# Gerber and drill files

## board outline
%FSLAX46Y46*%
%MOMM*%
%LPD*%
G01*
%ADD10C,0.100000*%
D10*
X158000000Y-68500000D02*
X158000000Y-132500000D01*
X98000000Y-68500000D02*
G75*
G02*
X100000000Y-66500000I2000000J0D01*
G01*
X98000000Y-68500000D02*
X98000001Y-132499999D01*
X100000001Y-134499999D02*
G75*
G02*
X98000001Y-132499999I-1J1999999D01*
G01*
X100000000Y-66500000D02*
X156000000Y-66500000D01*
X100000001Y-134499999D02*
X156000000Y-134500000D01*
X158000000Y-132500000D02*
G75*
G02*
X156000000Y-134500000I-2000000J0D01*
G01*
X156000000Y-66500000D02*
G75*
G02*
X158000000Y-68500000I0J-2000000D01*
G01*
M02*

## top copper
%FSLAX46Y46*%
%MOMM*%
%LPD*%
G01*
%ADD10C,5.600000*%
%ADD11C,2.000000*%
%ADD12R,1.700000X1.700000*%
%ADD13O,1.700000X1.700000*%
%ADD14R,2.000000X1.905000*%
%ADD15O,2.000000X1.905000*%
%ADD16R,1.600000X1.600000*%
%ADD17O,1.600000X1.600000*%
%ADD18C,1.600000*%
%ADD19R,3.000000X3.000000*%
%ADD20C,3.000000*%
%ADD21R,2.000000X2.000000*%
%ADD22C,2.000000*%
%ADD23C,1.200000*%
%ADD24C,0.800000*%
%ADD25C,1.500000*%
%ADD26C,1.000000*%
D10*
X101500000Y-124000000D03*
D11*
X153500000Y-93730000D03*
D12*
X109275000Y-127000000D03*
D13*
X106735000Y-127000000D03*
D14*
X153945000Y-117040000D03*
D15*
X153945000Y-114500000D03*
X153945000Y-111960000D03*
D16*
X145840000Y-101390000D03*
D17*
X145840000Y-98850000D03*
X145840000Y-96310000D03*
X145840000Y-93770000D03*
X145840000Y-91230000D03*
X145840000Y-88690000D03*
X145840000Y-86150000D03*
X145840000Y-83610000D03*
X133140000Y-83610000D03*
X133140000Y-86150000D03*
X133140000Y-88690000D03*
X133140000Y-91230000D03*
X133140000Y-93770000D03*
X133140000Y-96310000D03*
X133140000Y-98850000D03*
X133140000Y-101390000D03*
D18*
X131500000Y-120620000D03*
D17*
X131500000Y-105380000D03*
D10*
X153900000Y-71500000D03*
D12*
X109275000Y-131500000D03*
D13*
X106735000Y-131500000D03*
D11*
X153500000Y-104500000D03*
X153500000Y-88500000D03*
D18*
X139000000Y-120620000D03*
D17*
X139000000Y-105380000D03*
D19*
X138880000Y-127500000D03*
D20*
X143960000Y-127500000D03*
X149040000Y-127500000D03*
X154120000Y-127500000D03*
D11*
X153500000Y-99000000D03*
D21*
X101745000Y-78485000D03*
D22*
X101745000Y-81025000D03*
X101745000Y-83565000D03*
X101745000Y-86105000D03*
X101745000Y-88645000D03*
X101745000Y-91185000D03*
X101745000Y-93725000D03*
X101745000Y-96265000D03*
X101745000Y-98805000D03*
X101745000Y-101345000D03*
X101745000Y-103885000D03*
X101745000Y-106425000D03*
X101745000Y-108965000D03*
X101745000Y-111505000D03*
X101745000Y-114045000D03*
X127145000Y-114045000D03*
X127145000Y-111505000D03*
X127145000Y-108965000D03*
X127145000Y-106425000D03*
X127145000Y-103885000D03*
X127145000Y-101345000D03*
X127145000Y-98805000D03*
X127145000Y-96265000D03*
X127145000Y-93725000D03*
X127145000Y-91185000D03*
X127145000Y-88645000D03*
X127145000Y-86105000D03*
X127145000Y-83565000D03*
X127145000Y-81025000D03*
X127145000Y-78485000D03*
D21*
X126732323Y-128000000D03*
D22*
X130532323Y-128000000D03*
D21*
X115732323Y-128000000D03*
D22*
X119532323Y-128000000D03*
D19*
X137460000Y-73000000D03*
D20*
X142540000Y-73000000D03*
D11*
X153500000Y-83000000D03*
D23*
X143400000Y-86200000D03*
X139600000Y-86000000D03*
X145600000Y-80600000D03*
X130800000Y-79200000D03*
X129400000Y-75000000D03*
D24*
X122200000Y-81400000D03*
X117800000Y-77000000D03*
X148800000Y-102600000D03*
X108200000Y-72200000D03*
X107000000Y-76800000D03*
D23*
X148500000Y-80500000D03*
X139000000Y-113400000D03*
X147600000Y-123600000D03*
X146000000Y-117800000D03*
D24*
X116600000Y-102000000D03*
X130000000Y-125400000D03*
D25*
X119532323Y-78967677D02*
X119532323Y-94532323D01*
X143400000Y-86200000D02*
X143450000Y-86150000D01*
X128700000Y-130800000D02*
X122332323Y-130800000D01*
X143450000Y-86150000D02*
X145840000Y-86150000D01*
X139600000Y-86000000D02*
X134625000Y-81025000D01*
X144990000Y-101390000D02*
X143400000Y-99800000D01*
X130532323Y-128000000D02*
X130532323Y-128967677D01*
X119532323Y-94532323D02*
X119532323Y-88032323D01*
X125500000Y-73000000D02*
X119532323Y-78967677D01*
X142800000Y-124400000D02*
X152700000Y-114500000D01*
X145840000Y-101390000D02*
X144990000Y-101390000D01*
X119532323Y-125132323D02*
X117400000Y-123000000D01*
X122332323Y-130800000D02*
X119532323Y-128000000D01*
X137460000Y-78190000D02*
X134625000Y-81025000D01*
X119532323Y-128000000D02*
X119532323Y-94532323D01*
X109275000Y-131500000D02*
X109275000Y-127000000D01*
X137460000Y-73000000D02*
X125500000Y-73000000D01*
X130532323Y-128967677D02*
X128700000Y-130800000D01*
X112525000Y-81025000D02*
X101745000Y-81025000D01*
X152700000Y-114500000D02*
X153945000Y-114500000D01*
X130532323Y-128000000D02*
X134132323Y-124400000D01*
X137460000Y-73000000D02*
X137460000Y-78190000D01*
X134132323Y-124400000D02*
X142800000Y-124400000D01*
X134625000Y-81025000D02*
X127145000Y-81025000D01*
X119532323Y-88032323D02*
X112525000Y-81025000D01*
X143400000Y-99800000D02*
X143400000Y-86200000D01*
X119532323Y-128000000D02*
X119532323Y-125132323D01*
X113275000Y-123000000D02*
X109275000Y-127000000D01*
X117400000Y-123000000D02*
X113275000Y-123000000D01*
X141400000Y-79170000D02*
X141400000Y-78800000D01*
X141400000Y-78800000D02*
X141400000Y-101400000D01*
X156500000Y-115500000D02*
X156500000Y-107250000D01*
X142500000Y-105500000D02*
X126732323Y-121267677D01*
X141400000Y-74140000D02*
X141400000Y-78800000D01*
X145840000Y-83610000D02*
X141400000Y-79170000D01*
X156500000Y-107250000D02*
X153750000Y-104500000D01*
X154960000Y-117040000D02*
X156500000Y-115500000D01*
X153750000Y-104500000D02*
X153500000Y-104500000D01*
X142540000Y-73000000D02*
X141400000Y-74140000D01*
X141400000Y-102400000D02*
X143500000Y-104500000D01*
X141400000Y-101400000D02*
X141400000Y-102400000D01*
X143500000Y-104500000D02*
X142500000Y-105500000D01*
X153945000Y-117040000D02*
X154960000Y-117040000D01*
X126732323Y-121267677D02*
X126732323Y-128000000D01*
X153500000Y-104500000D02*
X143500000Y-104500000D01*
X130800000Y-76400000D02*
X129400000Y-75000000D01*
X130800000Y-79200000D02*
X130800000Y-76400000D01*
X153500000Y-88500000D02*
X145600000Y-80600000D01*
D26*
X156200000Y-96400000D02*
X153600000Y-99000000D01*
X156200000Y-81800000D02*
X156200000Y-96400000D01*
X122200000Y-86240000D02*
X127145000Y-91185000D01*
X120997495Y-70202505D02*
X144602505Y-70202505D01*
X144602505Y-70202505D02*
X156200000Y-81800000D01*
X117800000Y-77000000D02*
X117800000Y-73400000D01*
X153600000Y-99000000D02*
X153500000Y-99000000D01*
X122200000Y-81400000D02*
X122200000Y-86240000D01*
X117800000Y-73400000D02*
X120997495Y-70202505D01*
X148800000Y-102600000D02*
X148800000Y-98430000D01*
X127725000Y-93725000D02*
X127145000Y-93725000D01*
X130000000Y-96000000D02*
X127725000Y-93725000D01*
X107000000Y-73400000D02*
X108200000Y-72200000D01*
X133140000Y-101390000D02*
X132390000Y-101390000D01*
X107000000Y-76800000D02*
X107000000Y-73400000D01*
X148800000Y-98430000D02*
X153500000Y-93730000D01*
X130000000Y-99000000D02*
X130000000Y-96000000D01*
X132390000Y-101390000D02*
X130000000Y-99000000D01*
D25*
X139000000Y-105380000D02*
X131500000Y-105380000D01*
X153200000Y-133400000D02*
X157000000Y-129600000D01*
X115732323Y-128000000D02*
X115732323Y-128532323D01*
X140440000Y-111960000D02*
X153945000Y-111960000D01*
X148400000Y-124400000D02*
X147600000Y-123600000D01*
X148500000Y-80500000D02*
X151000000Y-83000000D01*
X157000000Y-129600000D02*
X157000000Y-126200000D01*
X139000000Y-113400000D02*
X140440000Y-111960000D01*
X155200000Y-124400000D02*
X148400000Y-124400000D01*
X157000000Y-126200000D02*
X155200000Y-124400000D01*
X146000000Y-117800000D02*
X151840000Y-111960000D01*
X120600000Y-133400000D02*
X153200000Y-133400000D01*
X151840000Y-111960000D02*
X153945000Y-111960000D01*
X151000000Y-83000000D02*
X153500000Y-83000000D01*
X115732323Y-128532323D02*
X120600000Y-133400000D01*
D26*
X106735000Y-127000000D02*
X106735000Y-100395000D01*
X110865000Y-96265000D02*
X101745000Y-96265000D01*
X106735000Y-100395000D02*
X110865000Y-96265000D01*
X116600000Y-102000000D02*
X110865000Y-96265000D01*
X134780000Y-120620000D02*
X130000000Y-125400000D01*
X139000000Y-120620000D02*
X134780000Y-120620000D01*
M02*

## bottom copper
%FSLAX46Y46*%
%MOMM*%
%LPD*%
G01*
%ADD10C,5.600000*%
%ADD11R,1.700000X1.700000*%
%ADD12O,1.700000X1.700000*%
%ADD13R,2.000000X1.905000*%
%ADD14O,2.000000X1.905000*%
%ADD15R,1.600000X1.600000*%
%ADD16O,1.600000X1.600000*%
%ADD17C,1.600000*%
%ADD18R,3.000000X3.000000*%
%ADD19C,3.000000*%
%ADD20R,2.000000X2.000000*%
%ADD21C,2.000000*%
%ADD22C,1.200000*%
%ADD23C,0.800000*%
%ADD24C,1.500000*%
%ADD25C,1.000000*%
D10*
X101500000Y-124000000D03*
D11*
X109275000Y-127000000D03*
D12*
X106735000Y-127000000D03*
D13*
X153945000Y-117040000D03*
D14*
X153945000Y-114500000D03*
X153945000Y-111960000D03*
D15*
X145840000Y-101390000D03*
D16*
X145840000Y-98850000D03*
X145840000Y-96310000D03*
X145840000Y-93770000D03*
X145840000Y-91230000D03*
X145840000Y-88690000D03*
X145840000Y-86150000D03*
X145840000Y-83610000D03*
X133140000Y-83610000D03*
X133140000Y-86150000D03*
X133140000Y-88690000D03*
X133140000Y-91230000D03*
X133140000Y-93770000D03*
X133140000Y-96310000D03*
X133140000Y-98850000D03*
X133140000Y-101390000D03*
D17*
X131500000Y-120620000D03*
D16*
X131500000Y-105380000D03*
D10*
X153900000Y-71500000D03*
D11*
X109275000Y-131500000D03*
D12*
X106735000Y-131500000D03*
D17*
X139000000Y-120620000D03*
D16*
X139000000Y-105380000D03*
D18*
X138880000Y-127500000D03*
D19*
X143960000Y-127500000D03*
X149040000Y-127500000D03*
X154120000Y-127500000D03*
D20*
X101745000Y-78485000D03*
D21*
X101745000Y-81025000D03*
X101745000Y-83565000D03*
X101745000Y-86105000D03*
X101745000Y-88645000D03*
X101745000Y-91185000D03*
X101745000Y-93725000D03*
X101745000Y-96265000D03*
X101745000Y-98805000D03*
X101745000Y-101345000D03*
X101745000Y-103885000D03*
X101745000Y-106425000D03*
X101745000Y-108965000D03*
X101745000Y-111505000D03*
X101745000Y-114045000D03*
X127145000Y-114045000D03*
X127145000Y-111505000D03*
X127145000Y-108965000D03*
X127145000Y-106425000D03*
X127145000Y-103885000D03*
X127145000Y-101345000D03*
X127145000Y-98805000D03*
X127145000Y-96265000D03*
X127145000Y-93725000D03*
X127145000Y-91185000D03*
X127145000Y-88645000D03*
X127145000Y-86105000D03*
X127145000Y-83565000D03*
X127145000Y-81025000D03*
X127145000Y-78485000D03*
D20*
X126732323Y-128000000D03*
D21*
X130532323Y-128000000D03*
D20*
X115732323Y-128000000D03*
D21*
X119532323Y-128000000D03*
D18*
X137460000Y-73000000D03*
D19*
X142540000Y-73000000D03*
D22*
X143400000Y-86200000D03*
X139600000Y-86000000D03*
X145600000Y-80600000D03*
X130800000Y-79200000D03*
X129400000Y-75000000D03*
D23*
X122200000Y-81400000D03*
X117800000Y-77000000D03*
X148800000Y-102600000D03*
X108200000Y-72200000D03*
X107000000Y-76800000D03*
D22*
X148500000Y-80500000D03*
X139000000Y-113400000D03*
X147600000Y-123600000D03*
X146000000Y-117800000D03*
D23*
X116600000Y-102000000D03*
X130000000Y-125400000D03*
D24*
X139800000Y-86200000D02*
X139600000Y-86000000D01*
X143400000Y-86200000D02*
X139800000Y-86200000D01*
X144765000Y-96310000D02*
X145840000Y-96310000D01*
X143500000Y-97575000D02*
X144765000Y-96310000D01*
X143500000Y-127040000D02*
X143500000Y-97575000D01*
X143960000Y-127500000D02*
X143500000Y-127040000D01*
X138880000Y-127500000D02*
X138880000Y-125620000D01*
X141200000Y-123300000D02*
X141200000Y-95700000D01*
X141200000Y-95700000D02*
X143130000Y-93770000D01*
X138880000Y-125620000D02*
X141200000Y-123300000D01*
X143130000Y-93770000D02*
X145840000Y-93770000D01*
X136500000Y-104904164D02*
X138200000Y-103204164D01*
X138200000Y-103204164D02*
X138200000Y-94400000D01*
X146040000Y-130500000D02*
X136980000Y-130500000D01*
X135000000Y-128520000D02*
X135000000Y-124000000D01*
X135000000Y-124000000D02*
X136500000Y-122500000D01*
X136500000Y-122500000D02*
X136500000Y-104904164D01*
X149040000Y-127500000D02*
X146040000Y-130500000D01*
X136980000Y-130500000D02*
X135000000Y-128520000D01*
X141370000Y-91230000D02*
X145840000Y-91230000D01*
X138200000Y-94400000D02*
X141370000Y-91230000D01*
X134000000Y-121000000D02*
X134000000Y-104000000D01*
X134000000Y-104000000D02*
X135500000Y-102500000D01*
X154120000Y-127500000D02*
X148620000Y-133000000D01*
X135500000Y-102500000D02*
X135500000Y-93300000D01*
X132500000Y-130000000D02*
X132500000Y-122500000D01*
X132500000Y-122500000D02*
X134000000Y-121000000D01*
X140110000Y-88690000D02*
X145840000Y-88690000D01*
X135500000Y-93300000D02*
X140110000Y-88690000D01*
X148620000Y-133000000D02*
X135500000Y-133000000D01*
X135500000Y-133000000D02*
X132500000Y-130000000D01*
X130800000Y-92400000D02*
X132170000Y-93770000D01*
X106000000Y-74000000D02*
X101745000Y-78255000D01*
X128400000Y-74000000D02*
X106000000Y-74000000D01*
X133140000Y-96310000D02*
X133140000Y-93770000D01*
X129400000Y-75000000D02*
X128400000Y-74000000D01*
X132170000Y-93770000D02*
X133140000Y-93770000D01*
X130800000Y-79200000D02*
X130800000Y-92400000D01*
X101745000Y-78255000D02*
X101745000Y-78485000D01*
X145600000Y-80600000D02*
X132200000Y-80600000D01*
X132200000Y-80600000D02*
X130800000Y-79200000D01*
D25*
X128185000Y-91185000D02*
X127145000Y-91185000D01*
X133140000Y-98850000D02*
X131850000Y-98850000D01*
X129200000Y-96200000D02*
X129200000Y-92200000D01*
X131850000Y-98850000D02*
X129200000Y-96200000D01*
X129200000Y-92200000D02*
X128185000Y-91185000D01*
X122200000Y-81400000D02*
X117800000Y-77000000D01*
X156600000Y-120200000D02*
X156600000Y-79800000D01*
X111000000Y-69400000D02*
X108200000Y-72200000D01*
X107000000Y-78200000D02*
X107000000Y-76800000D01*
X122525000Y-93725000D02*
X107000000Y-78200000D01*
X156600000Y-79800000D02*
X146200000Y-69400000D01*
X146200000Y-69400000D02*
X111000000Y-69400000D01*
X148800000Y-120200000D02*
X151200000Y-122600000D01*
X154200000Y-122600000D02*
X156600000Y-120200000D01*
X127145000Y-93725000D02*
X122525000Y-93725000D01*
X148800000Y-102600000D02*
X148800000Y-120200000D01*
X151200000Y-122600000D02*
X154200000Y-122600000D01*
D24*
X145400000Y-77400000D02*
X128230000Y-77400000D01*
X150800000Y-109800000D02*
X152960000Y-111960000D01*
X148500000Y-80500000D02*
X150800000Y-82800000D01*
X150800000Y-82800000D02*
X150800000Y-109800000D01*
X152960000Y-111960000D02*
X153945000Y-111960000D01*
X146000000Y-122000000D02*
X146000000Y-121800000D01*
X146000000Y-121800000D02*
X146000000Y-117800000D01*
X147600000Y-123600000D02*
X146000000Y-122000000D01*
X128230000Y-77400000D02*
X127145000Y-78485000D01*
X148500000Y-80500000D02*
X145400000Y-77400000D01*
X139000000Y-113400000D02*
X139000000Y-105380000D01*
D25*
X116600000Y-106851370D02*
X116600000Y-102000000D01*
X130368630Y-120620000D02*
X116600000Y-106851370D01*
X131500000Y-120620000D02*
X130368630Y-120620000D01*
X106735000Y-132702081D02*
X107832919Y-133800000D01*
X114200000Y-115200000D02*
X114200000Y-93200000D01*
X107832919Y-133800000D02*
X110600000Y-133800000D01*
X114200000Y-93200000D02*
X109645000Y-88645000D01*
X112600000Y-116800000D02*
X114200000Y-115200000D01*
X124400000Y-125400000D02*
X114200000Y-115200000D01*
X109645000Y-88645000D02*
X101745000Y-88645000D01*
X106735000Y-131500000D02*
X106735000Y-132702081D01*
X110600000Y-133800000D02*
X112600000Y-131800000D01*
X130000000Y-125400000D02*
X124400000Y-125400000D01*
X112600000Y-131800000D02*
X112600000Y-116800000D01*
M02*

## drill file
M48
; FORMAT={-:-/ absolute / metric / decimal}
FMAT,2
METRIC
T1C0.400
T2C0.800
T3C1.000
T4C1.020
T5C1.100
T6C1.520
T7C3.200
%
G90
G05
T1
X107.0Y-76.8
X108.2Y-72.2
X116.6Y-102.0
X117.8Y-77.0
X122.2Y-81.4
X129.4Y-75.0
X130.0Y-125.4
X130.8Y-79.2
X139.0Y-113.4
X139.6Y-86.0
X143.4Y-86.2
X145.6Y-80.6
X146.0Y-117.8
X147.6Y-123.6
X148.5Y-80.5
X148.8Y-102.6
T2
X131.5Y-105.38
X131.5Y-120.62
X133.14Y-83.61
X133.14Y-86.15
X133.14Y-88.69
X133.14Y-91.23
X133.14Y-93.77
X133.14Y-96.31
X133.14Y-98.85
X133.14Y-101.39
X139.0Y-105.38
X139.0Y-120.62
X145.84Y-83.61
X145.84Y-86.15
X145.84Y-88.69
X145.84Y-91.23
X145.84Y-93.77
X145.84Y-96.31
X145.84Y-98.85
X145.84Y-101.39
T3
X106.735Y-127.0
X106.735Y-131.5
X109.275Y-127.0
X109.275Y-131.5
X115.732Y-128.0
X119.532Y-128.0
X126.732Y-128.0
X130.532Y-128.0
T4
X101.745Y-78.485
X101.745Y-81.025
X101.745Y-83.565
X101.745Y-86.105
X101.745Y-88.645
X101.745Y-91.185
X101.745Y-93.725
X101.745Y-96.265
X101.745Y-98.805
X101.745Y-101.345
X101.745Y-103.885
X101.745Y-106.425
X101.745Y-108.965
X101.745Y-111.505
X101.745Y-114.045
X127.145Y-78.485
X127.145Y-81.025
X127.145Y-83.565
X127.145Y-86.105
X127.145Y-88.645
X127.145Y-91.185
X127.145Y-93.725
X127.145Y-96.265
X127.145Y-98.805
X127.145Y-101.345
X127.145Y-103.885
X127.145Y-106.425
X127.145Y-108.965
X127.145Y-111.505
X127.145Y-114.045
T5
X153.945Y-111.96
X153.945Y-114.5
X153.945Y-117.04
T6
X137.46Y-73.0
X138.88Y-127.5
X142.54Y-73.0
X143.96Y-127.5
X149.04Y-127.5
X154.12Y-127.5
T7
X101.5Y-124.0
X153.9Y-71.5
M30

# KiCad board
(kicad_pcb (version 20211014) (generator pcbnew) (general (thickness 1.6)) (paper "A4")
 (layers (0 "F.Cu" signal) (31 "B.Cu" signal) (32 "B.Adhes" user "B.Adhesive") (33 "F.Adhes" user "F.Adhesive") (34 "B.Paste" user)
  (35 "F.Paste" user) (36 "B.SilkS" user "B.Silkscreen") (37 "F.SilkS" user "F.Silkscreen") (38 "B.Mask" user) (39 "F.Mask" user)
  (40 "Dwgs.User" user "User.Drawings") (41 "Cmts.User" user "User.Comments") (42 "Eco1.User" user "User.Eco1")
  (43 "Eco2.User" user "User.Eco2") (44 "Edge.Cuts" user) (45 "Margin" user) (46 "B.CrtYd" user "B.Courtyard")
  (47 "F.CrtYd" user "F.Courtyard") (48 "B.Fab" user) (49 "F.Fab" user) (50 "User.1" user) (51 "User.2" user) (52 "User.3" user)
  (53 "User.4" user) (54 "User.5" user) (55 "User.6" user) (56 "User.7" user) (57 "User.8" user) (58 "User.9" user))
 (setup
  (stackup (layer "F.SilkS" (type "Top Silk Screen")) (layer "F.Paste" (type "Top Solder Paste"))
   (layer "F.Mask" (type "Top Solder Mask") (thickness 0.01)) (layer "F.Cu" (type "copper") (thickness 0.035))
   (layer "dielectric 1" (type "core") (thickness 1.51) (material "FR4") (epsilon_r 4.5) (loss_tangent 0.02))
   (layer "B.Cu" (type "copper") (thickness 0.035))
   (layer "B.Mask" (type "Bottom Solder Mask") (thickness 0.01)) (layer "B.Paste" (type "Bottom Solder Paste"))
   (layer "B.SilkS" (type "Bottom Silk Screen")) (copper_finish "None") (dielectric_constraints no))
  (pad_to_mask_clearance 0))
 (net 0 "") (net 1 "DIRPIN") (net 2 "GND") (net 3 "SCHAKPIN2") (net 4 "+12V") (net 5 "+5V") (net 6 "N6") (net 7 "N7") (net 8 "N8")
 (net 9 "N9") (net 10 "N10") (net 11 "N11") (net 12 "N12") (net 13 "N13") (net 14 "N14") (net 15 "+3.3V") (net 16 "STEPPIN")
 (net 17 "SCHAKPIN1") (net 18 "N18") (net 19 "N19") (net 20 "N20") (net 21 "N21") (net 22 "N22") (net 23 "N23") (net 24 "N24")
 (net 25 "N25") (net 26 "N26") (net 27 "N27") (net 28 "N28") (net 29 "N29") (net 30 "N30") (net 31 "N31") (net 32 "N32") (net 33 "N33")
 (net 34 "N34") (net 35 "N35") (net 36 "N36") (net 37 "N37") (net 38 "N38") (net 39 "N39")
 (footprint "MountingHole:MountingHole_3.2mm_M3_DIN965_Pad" (layer "F.Cu") (at 101.5 124)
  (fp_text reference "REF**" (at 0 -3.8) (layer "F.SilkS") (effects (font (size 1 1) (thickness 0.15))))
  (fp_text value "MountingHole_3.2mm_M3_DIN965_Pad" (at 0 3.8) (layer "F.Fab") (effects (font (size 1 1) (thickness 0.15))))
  (pad "1" thru_hole circle (at 0 0) (size 5.6 5.6) (drill 3.2) (layers *.Cu *.Mask)))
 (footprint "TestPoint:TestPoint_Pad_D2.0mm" (layer "F.Cu") (at 153.5 93.73)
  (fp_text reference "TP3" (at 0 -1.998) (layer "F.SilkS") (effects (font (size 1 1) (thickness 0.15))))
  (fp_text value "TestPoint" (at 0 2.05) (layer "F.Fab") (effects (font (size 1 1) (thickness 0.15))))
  (pad "1" smd circle (at 0 0) (size 2 2) (layers "F.Cu" "F.Mask") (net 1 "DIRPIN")))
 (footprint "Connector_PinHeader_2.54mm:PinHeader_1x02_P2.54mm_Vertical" (layer "F.Cu") (at 109.275 127 -90)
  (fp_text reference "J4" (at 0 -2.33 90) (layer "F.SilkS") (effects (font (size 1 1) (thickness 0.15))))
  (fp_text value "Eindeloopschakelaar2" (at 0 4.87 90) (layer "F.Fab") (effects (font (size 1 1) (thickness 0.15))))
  (pad "1" thru_hole rect (at 0 0 270) (size 1.7 1.7) (drill 1) (layers *.Cu *.Mask) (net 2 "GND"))
  (pad "2" thru_hole oval (at 0 2.54 270) (size 1.7 1.7) (drill 1) (layers *.Cu *.Mask) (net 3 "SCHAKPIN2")))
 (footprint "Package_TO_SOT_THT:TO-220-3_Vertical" (layer "F.Cu") (at 153.945 117.04 90)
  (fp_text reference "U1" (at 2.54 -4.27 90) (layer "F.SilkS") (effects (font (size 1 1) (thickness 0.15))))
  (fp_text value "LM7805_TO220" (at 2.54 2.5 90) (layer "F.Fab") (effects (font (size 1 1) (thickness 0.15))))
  (pad "1" thru_hole rect (at 0 0 90) (size 1.905 2) (drill 1.1) (layers *.Cu *.Mask) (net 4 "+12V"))
  (pad "2" thru_hole oval (at 2.54 0 90) (size 1.905 2) (drill 1.1) (layers *.Cu *.Mask) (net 2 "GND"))
  (pad "3" thru_hole oval (at 5.08 0 90) (size 1.905 2) (drill 1.1) (layers *.Cu *.Mask) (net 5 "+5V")))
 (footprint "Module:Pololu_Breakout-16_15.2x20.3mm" (layer "F.Cu") (at 145.84 101.39 180)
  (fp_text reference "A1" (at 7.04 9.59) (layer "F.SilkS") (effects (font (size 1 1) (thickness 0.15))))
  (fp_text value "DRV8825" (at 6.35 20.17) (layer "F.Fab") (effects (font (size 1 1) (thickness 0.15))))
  (pad "1" thru_hole rect (at 0 0 180) (size 1.6 1.6) (drill 0.8) (layers *.Cu *.Mask) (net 2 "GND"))
  (pad "2" thru_hole oval (at 0 2.54 180) (size 1.6 1.6) (drill 0.8) (layers *.Cu *.Mask) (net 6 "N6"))
  (pad "3" thru_hole oval (at 0 5.08 180) (size 1.6 1.6) (drill 0.8) (layers *.Cu *.Mask) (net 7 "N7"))
  (pad "4" thru_hole oval (at 0 7.62 180) (size 1.6 1.6) (drill 0.8) (layers *.Cu *.Mask) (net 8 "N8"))
  (pad "5" thru_hole oval (at 0 10.16 180) (size 1.6 1.6) (drill 0.8) (layers *.Cu *.Mask) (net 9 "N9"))
  (pad "6" thru_hole oval (at 0 12.7 180) (size 1.6 1.6) (drill 0.8) (layers *.Cu *.Mask) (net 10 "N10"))
  (pad "7" thru_hole oval (at 0 15.24 180) (size 1.6 1.6) (drill 0.8) (layers *.Cu *.Mask) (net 2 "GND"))
  (pad "8" thru_hole oval (at 0 17.78 180) (size 1.6 1.6) (drill 0.8) (layers *.Cu *.Mask) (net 4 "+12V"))
  (pad "9" thru_hole oval (at 12.7 17.78 180) (size 1.6 1.6) (drill 0.8) (layers *.Cu *.Mask) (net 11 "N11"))
  (pad "10" thru_hole oval (at 12.7 15.24 180) (size 1.6 1.6) (drill 0.8) (layers *.Cu *.Mask) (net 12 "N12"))
  (pad "11" thru_hole oval (at 12.7 12.7 180) (size 1.6 1.6) (drill 0.8) (layers *.Cu *.Mask) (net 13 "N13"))
  (pad "12" thru_hole oval (at 12.7 10.16 180) (size 1.6 1.6) (drill 0.8) (layers *.Cu *.Mask) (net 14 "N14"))
  (pad "13" thru_hole oval (at 12.7 7.62 180) (size 1.6 1.6) (drill 0.8) (layers *.Cu *.Mask) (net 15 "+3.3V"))
  (pad "14" thru_hole oval (at 12.7 5.08 180) (size 1.6 1.6) (drill 0.8) (layers *.Cu *.Mask) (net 15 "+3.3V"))
  (pad "15" thru_hole oval (at 12.7 2.54 180) (size 1.6 1.6) (drill 0.8) (layers *.Cu *.Mask) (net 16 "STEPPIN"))
  (pad "16" thru_hole oval (at 12.7 0 180) (size 1.6 1.6) (drill 0.8) (layers *.Cu *.Mask) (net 1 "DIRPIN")))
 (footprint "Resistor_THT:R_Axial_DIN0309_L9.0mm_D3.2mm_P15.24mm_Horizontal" (layer "F.Cu") (at 131.5 120.62 90)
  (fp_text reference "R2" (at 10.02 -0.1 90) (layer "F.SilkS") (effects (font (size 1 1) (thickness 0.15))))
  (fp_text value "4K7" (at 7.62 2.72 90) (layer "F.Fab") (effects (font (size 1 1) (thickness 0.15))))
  (pad "1" thru_hole circle (at 0 0 90) (size 1.6 1.6) (drill 0.8) (layers *.Cu *.Mask) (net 3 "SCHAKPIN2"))
  (pad "2" thru_hole oval (at 15.24 0 90) (size 1.6 1.6) (drill 0.8) (layers *.Cu *.Mask) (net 5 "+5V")))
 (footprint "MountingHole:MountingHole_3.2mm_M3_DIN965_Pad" (layer "F.Cu") (at 153.9 71.5)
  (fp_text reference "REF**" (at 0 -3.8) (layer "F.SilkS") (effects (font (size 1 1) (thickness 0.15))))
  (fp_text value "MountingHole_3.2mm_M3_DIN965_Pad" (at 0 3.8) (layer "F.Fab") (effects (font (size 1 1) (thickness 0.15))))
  (pad "1" thru_hole circle (at 0 0) (size 5.6 5.6) (drill 3.2) (layers *.Cu *.Mask)))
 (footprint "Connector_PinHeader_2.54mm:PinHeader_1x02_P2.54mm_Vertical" (layer "F.Cu") (at 109.275 131.5 -90)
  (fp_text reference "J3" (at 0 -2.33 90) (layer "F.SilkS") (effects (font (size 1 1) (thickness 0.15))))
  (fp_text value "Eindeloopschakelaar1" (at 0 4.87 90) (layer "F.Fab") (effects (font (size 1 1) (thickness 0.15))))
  (pad "1" thru_hole rect (at 0 0 270) (size 1.7 1.7) (drill 1) (layers *.Cu *.Mask) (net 2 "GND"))
  (pad "2" thru_hole oval (at 0 2.54 270) (size 1.7 1.7) (drill 1) (layers *.Cu *.Mask) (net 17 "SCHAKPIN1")))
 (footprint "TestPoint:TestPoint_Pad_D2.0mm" (layer "F.Cu") (at 153.5 104.5)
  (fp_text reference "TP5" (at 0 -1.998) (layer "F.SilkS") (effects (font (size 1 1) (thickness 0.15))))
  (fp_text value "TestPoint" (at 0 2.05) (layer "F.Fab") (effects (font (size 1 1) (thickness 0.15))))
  (pad "1" smd circle (at 0 0) (size 2 2) (layers "F.Cu" "F.Mask") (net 4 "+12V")))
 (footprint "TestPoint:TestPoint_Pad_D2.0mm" (layer "F.Cu") (at 153.5 88.5)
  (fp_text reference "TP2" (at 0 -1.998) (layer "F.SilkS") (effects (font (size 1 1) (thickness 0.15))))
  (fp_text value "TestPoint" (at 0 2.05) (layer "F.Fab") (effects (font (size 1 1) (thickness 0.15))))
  (pad "1" smd circle (at 0 0) (size 2 2) (layers "F.Cu" "F.Mask") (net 15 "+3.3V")))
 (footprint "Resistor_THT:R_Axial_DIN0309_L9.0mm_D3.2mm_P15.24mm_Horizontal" (layer "F.Cu") (at 139 120.62 90)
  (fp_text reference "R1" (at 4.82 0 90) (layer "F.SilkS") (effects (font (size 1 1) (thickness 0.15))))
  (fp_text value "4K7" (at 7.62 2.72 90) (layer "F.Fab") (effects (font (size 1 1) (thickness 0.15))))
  (pad "1" thru_hole circle (at 0 0 90) (size 1.6 1.6) (drill 0.8) (layers *.Cu *.Mask) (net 17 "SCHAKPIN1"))
  (pad "2" thru_hole oval (at 15.24 0 90) (size 1.6 1.6) (drill 0.8) (layers *.Cu *.Mask) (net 5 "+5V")))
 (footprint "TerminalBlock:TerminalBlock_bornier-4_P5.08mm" (layer "F.Cu") (at 138.88 127.5)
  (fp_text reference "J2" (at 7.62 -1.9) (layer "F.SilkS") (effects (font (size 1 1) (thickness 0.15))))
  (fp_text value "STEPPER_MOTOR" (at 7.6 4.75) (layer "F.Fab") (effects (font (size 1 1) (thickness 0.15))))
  (pad "1" thru_hole rect (at 0 0) (size 3 3) (drill 1.52) (layers *.Cu *.Mask) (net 8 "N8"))
  (pad "2" thru_hole circle (at 5.08 0) (size 3 3) (drill 1.52) (layers *.Cu *.Mask) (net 7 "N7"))
  (pad "3" thru_hole circle (at 10.16 0) (size 3 3) (drill 1.52) (layers *.Cu *.Mask) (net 9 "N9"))
  (pad "4" thru_hole circle (at 15.24 0) (size 3 3) (drill 1.52) (layers *.Cu *.Mask) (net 10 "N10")))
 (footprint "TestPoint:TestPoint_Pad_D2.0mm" (layer "F.Cu") (at 153.5 99)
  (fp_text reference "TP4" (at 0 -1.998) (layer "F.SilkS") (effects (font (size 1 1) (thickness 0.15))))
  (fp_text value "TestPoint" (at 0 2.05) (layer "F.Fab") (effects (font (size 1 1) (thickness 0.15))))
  (pad "1" smd circle (at 0 0) (size 2 2) (layers "F.Cu" "F.Mask") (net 16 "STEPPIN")))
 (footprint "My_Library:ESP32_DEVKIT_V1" (layer "F.Cu") (at 114.445 94)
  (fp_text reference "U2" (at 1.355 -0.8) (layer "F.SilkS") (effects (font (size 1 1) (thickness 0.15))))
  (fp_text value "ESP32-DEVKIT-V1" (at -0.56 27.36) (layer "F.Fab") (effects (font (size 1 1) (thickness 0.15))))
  (pad "1" thru_hole rect (at -12.7 -15.515) (size 2 2) (drill 1.02) (layers *.Cu *.Mask) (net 15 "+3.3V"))
  (pad "2" thru_hole circle (at -12.7 -12.975) (size 2 2) (drill 1.02) (layers *.Cu *.Mask) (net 2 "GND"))
  (pad "3" thru_hole circle (at -12.7 -10.435) (size 2 2) (drill 1.02) (layers *.Cu *.Mask) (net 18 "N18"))
  (pad "4" thru_hole circle (at -12.7 -7.895) (size 2 2) (drill 1.02) (layers *.Cu *.Mask) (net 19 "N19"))
  (pad "5" thru_hole circle (at -12.7 -5.355) (size 2 2) (drill 1.02) (layers *.Cu *.Mask) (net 17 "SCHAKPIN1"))
  (pad "6" thru_hole circle (at -12.7 -2.815) (size 2 2) (drill 1.02) (layers *.Cu *.Mask) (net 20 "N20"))
  (pad "7" thru_hole circle (at -12.7 -0.275) (size 2 2) (drill 1.02) (layers *.Cu *.Mask) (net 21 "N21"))
  (pad "8" thru_hole circle (at -12.7 2.265) (size 2 2) (drill 1.02) (layers *.Cu *.Mask) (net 3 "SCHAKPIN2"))
  (pad "9" thru_hole circle (at -12.7 4.805) (size 2 2) (drill 1.02) (layers *.Cu *.Mask) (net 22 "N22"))
  (pad "10" thru_hole circle (at -12.7 7.345) (size 2 2) (drill 1.02) (layers *.Cu *.Mask) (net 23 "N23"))
  (pad "11" thru_hole circle (at -12.7 9.885) (size 2 2) (drill 1.02) (layers *.Cu *.Mask) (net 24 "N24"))
  (pad "12" thru_hole circle (at -12.7 12.425) (size 2 2) (drill 1.02) (layers *.Cu *.Mask) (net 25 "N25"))
  (pad "13" thru_hole circle (at -12.7 14.965) (size 2 2) (drill 1.02) (layers *.Cu *.Mask) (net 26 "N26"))
  (pad "14" thru_hole circle (at -12.7 17.505) (size 2 2) (drill 1.02) (layers *.Cu *.Mask) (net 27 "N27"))
  (pad "15" thru_hole circle (at -12.7 20.045) (size 2 2) (drill 1.02) (layers *.Cu *.Mask) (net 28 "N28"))
  (pad "16" thru_hole circle (at 12.7 20.045) (size 2 2) (drill 1.02) (layers *.Cu *.Mask) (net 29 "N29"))
  (pad "17" thru_hole circle (at 12.7 17.505) (size 2 2) (drill 1.02) (layers *.Cu *.Mask) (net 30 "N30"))
  (pad "18" thru_hole circle (at 12.7 14.965) (size 2 2) (drill 1.02) (layers *.Cu *.Mask) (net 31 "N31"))
  (pad "19" thru_hole circle (at 12.7 12.425) (size 2 2) (drill 1.02) (layers *.Cu *.Mask) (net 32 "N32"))
  (pad "20" thru_hole circle (at 12.7 9.885) (size 2 2) (drill 1.02) (layers *.Cu *.Mask) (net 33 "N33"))
  (pad "21" thru_hole circle (at 12.7 7.345) (size 2 2) (drill 1.02) (layers *.Cu *.Mask) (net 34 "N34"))
  (pad "22" thru_hole circle (at 12.7 4.805) (size 2 2) (drill 1.02) (layers *.Cu *.Mask) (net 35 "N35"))
  (pad "23" thru_hole circle (at 12.7 2.265) (size 2 2) (drill 1.02) (layers *.Cu *.Mask) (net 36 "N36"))
  (pad "24" thru_hole circle (at 12.7 -0.275) (size 2 2) (drill 1.02) (layers *.Cu *.Mask) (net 1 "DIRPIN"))
  (pad "25" thru_hole circle (at 12.7 -2.815) (size 2 2) (drill 1.02) (layers *.Cu *.Mask) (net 16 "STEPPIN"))
  (pad "26" thru_hole circle (at 12.7 -5.355) (size 2 2) (drill 1.02) (layers *.Cu *.Mask) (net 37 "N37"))
  (pad "27" thru_hole circle (at 12.7 -7.895) (size 2 2) (drill 1.02) (layers *.Cu *.Mask) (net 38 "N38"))
  (pad "28" thru_hole circle (at 12.7 -10.435) (size 2 2) (drill 1.02) (layers *.Cu *.Mask) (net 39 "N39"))
  (pad "29" thru_hole circle (at 12.7 -12.975) (size 2 2) (drill 1.02) (layers *.Cu *.Mask) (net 2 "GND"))
  (pad "30" thru_hole circle (at 12.7 -15.515) (size 2 2) (drill 1.02) (layers *.Cu *.Mask) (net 5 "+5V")))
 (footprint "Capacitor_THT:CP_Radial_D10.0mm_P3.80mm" (layer "F.Cu") (at 126.732323 128)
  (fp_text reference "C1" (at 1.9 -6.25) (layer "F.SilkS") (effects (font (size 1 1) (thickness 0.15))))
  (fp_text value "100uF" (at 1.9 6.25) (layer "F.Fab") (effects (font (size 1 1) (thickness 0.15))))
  (pad "1" thru_hole rect (at 0 0) (size 2 2) (drill 1) (layers *.Cu *.Mask) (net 4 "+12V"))
  (pad "2" thru_hole circle (at 3.8 0) (size 2 2) (drill 1) (layers *.Cu *.Mask) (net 2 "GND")))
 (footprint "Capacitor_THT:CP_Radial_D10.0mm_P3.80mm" (layer "F.Cu") (at 115.732323 128)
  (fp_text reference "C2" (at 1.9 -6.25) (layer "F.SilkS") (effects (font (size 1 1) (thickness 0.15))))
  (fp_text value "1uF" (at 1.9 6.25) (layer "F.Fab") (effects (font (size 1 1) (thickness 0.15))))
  (pad "1" thru_hole rect (at 0 0) (size 2 2) (drill 1) (layers *.Cu *.Mask) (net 5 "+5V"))
  (pad "2" thru_hole circle (at 3.8 0) (size 2 2) (drill 1) (layers *.Cu *.Mask) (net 2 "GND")))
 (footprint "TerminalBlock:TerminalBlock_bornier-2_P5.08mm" (layer "F.Cu") (at 137.46 73)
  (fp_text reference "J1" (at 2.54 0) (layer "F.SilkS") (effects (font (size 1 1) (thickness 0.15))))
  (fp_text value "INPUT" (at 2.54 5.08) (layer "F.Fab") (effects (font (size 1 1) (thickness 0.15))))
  (pad "1" thru_hole rect (at 0 0) (size 3 3) (drill 1.52) (layers *.Cu *.Mask) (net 2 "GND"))
  (pad "2" thru_hole circle (at 5.08 0) (size 3 3) (drill 1.52) (layers *.Cu *.Mask) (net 4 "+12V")))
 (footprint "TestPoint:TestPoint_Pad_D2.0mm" (layer "F.Cu") (at 153.5 83)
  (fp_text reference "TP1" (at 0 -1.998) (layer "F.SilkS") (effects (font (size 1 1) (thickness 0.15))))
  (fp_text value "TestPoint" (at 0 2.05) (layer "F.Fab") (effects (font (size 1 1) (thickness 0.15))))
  (pad "1" smd circle (at 0 0) (size 2 2) (layers "F.Cu" "F.Mask") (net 5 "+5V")))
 (gr_line (start 158 68.5) (end 158 132.5) (layer "Edge.Cuts") (width 0.1))
 (gr_arc (start 98 68.5) (mid 98.585786 67.085786) (end 100 66.5) (layer "Edge.Cuts") (width 0.1))
 (gr_line (start 98 68.5) (end 98.000001 132.499999) (layer "Edge.Cuts") (width 0.1))
 (gr_arc (start 100.000001 134.499999) (mid 98.585787 133.914213) (end 98.000001 132.499999) (layer "Edge.Cuts") (width 0.1))
 (gr_line (start 100 66.5) (end 156 66.5) (layer "Edge.Cuts") (width 0.1))
 (gr_line (start 100.000001 134.499999) (end 156 134.5) (layer "Edge.Cuts") (width 0.1))
 (gr_arc (start 158 132.5) (mid 157.414214 133.914214) (end 156 134.5) (layer "Edge.Cuts") (width 0.1))
 (gr_arc (start 156 66.5) (mid 157.414214 67.085786) (end 158 68.5) (layer "Edge.Cuts") (width 0.1))
 (segment (start 119.532323 78.967677) (end 119.532323 94.532323) (width 1.5) (layer "F.Cu") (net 2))
 (segment (start 143.4 86.2) (end 143.45 86.15) (width 1.5) (layer "F.Cu") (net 2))
 (segment (start 128.7 130.8) (end 122.332323 130.8) (width 1.5) (layer "F.Cu") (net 2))
 (segment (start 143.45 86.15) (end 145.84 86.15) (width 1.5) (layer "F.Cu") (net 2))
 (segment (start 139.6 86) (end 134.625 81.025) (width 1.5) (layer "F.Cu") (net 2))
 (segment (start 144.99 101.39) (end 143.4 99.8) (width 1.5) (layer "F.Cu") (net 2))
 (segment (start 130.532323 128) (end 130.532323 128.967677) (width 1.5) (layer "F.Cu") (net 2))
 (segment (start 119.532323 94.532323) (end 119.532323 88.032323) (width 1.5) (layer "F.Cu") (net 2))
 (segment (start 125.5 73) (end 119.532323 78.967677) (width 1.5) (layer "F.Cu") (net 2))
 (segment (start 142.8 124.4) (end 152.7 114.5) (width 1.5) (layer "F.Cu") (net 2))
 (segment (start 145.84 101.39) (end 144.99 101.39) (width 1.5) (layer "F.Cu") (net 2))
 (segment (start 119.532323 125.132323) (end 117.4 123) (width 1.5) (layer "F.Cu") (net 2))
 (segment (start 122.332323 130.8) (end 119.532323 128) (width 1.5) (layer "F.Cu") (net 2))
 (segment (start 137.46 78.19) (end 134.625 81.025) (width 1.5) (layer "F.Cu") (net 2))
 (segment (start 119.532323 128) (end 119.532323 94.532323) (width 1.5) (layer "F.Cu") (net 2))
 (segment (start 109.275 131.5) (end 109.275 127) (width 1.5) (layer "F.Cu") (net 2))
 (segment (start 137.46 73) (end 125.5 73) (width 1.5) (layer "F.Cu") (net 2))
 (segment (start 130.532323 128.967677) (end 128.7 130.8) (width 1.5) (layer "F.Cu") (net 2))
 (segment (start 112.525 81.025) (end 101.745 81.025) (width 1.5) (layer "F.Cu") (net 2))
 (segment (start 152.7 114.5) (end 153.945 114.5) (width 1.5) (layer "F.Cu") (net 2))
 (segment (start 130.532323 128) (end 134.132323 124.4) (width 1.5) (layer "F.Cu") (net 2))
 (segment (start 137.46 73) (end 137.46 78.19) (width 1.5) (layer "F.Cu") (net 2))
 (segment (start 134.132323 124.4) (end 142.8 124.4) (width 1.5) (layer "F.Cu") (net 2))
 (segment (start 134.625 81.025) (end 127.145 81.025) (width 1.5) (layer "F.Cu") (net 2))
 (segment (start 119.532323 88.032323) (end 112.525 81.025) (width 1.5) (layer "F.Cu") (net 2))
 (segment (start 143.4 99.8) (end 143.4 86.2) (width 1.5) (layer "F.Cu") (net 2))
 (segment (start 119.532323 128) (end 119.532323 125.132323) (width 1.5) (layer "F.Cu") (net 2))
 (segment (start 113.275 123) (end 109.275 127) (width 1.5) (layer "F.Cu") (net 2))
 (segment (start 117.4 123) (end 113.275 123) (width 1.5) (layer "F.Cu") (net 2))
 (via (at 143.4 86.2) (size 1.2) (drill 0.4) (layers "F.Cu" "B.Cu") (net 2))
 (via (at 139.6 86) (size 1.2) (drill 0.4) (layers "F.Cu" "B.Cu") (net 2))
 (segment (start 139.8 86.2) (end 139.6 86) (width 1.5) (layer "B.Cu") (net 2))
 (segment (start 143.4 86.2) (end 139.8 86.2) (width 1.5) (layer "B.Cu") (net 2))
 (segment (start 144.765 96.31) (end 145.84 96.31) (width 1.5) (layer "B.Cu") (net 7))
 (segment (start 143.5 97.575) (end 144.765 96.31) (width 1.5) (layer "B.Cu") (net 7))
 (segment (start 143.5 127.04) (end 143.5 97.575) (width 1.5) (layer "B.Cu") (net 7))
 (segment (start 143.96 127.5) (end 143.5 127.04) (width 1.5) (layer "B.Cu") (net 7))
 (segment (start 138.88 127.5) (end 138.88 125.62) (width 1.5) (layer "B.Cu") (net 8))
 (segment (start 141.2 123.3) (end 141.2 95.7) (width 1.5) (layer "B.Cu") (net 8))
 (segment (start 141.2 95.7) (end 143.13 93.77) (width 1.5) (layer "B.Cu") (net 8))
 (segment (start 138.88 125.62) (end 141.2 123.3) (width 1.5) (layer "B.Cu") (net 8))
 (segment (start 143.13 93.77) (end 145.84 93.77) (width 1.5) (layer "B.Cu") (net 8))
 (segment (start 136.5 104.904164) (end 138.2 103.204164) (width 1.5) (layer "B.Cu") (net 9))
 (segment (start 138.2 103.204164) (end 138.2 94.4) (width 1.5) (layer "B.Cu") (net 9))
 (segment (start 146.04 130.5) (end 136.98 130.5) (width 1.5) (layer "B.Cu") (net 9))
 (segment (start 135 128.52) (end 135 124) (width 1.5) (layer "B.Cu") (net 9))
 (segment (start 135 124) (end 136.5 122.5) (width 1.5) (layer "B.Cu") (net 9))
 (segment (start 136.5 122.5) (end 136.5 104.904164) (width 1.5) (layer "B.Cu") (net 9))
 (segment (start 149.04 127.5) (end 146.04 130.5) (width 1.5) (layer "B.Cu") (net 9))
 (segment (start 136.98 130.5) (end 135 128.52) (width 1.5) (layer "B.Cu") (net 9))
 (segment (start 141.37 91.23) (end 145.84 91.23) (width 1.5) (layer "B.Cu") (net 9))
 (segment (start 138.2 94.4) (end 141.37 91.23) (width 1.5) (layer "B.Cu") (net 9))
 (segment (start 134 121) (end 134 104) (width 1.5) (layer "B.Cu") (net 10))
 (segment (start 134 104) (end 135.5 102.5) (width 1.5) (layer "B.Cu") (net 10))
 (segment (start 154.12 127.5) (end 148.62 133) (width 1.5) (layer "B.Cu") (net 10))
 (segment (start 135.5 102.5) (end 135.5 93.3) (width 1.5) (layer "B.Cu") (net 10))
 (segment (start 132.5 130) (end 132.5 122.5) (width 1.5) (layer "B.Cu") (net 10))
 (segment (start 132.5 122.5) (end 134 121) (width 1.5) (layer "B.Cu") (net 10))
 (segment (start 140.11 88.69) (end 145.84 88.69) (width 1.5) (layer "B.Cu") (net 10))
 (segment (start 135.5 93.3) (end 140.11 88.69) (width 1.5) (layer "B.Cu") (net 10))
 (segment (start 148.62 133) (end 135.5 133) (width 1.5) (layer "B.Cu") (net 10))
 (segment (start 135.5 133) (end 132.5 130) (width 1.5) (layer "B.Cu") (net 10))
 (segment (start 141.4 79.17) (end 141.4 78.8) (width 1.5) (layer "F.Cu") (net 4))
 (segment (start 141.4 78.8) (end 141.4 101.4) (width 1.5) (layer "F.Cu") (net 4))
 (segment (start 156.5 115.5) (end 156.5 107.25) (width 1.5) (layer "F.Cu") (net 4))
 (segment (start 142.5 105.5) (end 126.732323 121.267677) (width 1.5) (layer "F.Cu") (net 4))
 (segment (start 141.4 74.14) (end 141.4 78.8) (width 1.5) (layer "F.Cu") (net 4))
 (segment (start 145.84 83.61) (end 141.4 79.17) (width 1.5) (layer "F.Cu") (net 4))
 (segment (start 156.5 107.25) (end 153.75 104.5) (width 1.5) (layer "F.Cu") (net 4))
 (segment (start 154.96 117.04) (end 156.5 115.5) (width 1.5) (layer "F.Cu") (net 4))
 (segment (start 153.75 104.5) (end 153.5 104.5) (width 1.5) (layer "F.Cu") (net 4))
 (segment (start 142.54 73) (end 141.4 74.14) (width 1.5) (layer "F.Cu") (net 4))
 (segment (start 141.4 102.4) (end 143.5 104.5) (width 1.5) (layer "F.Cu") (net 4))
 (segment (start 141.4 101.4) (end 141.4 102.4) (width 1.5) (layer "F.Cu") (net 4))
 (segment (start 143.5 104.5) (end 142.5 105.5) (width 1.5) (layer "F.Cu") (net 4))
 (segment (start 153.945 117.04) (end 154.96 117.04) (width 1.5) (layer "F.Cu") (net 4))
 (segment (start 126.732323 121.267677) (end 126.732323 128) (width 1.5) (layer "F.Cu") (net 4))
 (segment (start 153.5 104.5) (end 143.5 104.5) (width 1.5) (layer "F.Cu") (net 4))
 (segment (start 130.8 76.4) (end 129.4 75) (width 1.5) (layer "F.Cu") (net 15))
 (segment (start 130.8 79.2) (end 130.8 76.4) (width 1.5) (layer "F.Cu") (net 15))
 (segment (start 153.5 88.5) (end 145.6 80.6) (width 1.5) (layer "F.Cu") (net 15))
 (via (at 145.6 80.6) (size 1.2) (drill 0.4) (layers "F.Cu" "B.Cu") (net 15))
 (via (at 130.8 79.2) (size 1.2) (drill 0.4) (layers "F.Cu" "B.Cu") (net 15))
 (via (at 129.4 75) (size 1.2) (drill 0.4) (layers "F.Cu" "B.Cu") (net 15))
 (segment (start 130.8 92.4) (end 132.17 93.77) (width 1.5) (layer "B.Cu") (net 15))
 (segment (start 106 74) (end 101.745 78.255) (width 1.5) (layer "B.Cu") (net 15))
 (segment (start 128.4 74) (end 106 74) (width 1.5) (layer "B.Cu") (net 15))
 (segment (start 133.14 96.31) (end 133.14 93.77) (width 1.5) (layer "B.Cu") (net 15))
 (segment (start 129.4 75) (end 128.4 74) (width 1.5) (layer "B.Cu") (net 15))
 (segment (start 132.17 93.77) (end 133.14 93.77) (width 1.5) (layer "B.Cu") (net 15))
 (segment (start 130.8 79.2) (end 130.8 92.4) (width 1.5) (layer "B.Cu") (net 15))
 (segment (start 101.745 78.255) (end 101.745 78.485) (width 1.5) (layer "B.Cu") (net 15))
 (segment (start 145.6 80.6) (end 132.2 80.6) (width 1.5) (layer "B.Cu") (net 15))
 (segment (start 132.2 80.6) (end 130.8 79.2) (width 1.5) (layer "B.Cu") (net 15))
 (segment (start 156.2 96.4) (end 153.6 99) (width 1) (layer "F.Cu") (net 16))
 (segment (start 156.2 81.8) (end 156.2 96.4) (width 1) (layer "F.Cu") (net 16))
 (segment (start 122.2 86.24) (end 127.145 91.185) (width 1) (layer "F.Cu") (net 16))
 (segment (start 120.997495 70.202505) (end 144.602505 70.202505) (width 1) (layer "F.Cu") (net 16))
 (segment (start 144.602505 70.202505) (end 156.2 81.8) (width 1) (layer "F.Cu") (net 16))
 (segment (start 117.8 77) (end 117.8 73.4) (width 1) (layer "F.Cu") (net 16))
 (segment (start 153.6 99) (end 153.5 99) (width 1) (layer "F.Cu") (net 16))
 (segment (start 122.2 81.4) (end 122.2 86.24) (width 1) (layer "F.Cu") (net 16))
 (segment (start 117.8 73.4) (end 120.997495 70.202505) (width 1) (layer "F.Cu") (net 16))
 (via (at 122.2 81.4) (size 0.8) (drill 0.4) (layers "F.Cu" "B.Cu") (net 16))
 (via (at 117.8 77) (size 0.8) (drill 0.4) (layers "F.Cu" "B.Cu") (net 16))
 (segment (start 128.185 91.185) (end 127.145 91.185) (width 1) (layer "B.Cu") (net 16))
 (segment (start 133.14 98.85) (end 131.85 98.85) (width 1) (layer "B.Cu") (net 16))
 (segment (start 129.2 96.2) (end 129.2 92.2) (width 1) (layer "B.Cu") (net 16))
 (segment (start 131.85 98.85) (end 129.2 96.2) (width 1) (layer "B.Cu") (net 16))
 (segment (start 129.2 92.2) (end 128.185 91.185) (width 1) (layer "B.Cu") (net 16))
 (segment (start 122.2 81.4) (end 117.8 77) (width 1) (layer "B.Cu") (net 16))
 (segment (start 148.8 102.6) (end 148.8 98.43) (width 1) (layer "F.Cu") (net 1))
 (segment (start 127.725 93.725) (end 127.145 93.725) (width 1) (layer "F.Cu") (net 1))
 (segment (start 130 96) (end 127.725 93.725) (width 1) (layer "F.Cu") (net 1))
 (segment (start 107 73.4) (end 108.2 72.2) (width 1) (layer "F.Cu") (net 1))
 (segment (start 133.14 101.39) (end 132.39 101.39) (width 1) (layer "F.Cu") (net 1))
 (segment (start 107 76.8) (end 107 73.4) (width 1) (layer "F.Cu") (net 1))
 (segment (start 148.8 98.43) (end 153.5 93.73) (width 1) (layer "F.Cu") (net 1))
 (segment (start 130 99) (end 130 96) (width 1) (layer "F.Cu") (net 1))
 (segment (start 132.39 101.39) (end 130 99) (width 1) (layer "F.Cu") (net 1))
 (via (at 148.8 102.6) (size 0.8) (drill 0.4) (layers "F.Cu" "B.Cu") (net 1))
 (via (at 108.2 72.2) (size 0.8) (drill 0.4) (layers "F.Cu" "B.Cu") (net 1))
 (via (at 107 76.8) (size 0.8) (drill 0.4) (layers "F.Cu" "B.Cu") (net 1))
 (segment (start 156.6 120.2) (end 156.6 79.8) (width 1) (layer "B.Cu") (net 1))
 (segment (start 111 69.4) (end 108.2 72.2) (width 1) (layer "B.Cu") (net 1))
 (segment (start 107 78.2) (end 107 76.8) (width 1) (layer "B.Cu") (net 1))
 (segment (start 122.525 93.725) (end 107 78.2) (width 1) (layer "B.Cu") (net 1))
 (segment (start 156.6 79.8) (end 146.2 69.4) (width 1) (layer "B.Cu") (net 1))
 (segment (start 146.2 69.4) (end 111 69.4) (width 1) (layer "B.Cu") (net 1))
 (segment (start 148.8 120.2) (end 151.2 122.6) (width 1) (layer "B.Cu") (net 1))
 (segment (start 154.2 122.6) (end 156.6 120.2) (width 1) (layer "B.Cu") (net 1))
 (segment (start 127.145 93.725) (end 122.525 93.725) (width 1) (layer "B.Cu") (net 1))
 (segment (start 148.8 102.6) (end 148.8 120.2) (width 1) (layer "B.Cu") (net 1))
 (segment (start 151.2 122.6) (end 154.2 122.6) (width 1) (layer "B.Cu") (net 1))
 (segment (start 139 105.38) (end 131.5 105.38) (width 1.5) (layer "F.Cu") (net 5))
 (segment (start 153.2 133.4) (end 157 129.6) (width 1.5) (layer "F.Cu") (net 5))
 (segment (start 115.732323 128) (end 115.732323 128.532323) (width 1.5) (layer "F.Cu") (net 5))
 (segment (start 140.44 111.96) (end 153.945 111.96) (width 1.5) (layer "F.Cu") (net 5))
 (segment (start 148.4 124.4) (end 147.6 123.6) (width 1.5) (layer "F.Cu") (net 5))
 (segment (start 148.5 80.5) (end 151 83) (width 1.5) (layer "F.Cu") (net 5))
 (segment (start 157 129.6) (end 157 126.2) (width 1.5) (layer "F.Cu") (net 5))
 (segment (start 139 113.4) (end 140.44 111.96) (width 1.5) (layer "F.Cu") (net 5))
 (segment (start 155.2 124.4) (end 148.4 124.4) (width 1.5) (layer "F.Cu") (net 5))
 (segment (start 157 126.2) (end 155.2 124.4) (width 1.5) (layer "F.Cu") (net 5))
 (segment (start 146 117.8) (end 151.84 111.96) (width 1.5) (layer "F.Cu") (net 5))
 (segment (start 120.6 133.4) (end 153.2 133.4) (width 1.5) (layer "F.Cu") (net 5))
 (segment (start 151.84 111.96) (end 153.945 111.96) (width 1.5) (layer "F.Cu") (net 5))
 (segment (start 151 83) (end 153.5 83) (width 1.5) (layer "F.Cu") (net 5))
 (segment (start 115.732323 128.532323) (end 120.6 133.4) (width 1.5) (layer "F.Cu") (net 5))
 (via (at 148.5 80.5) (size 1.2) (drill 0.4) (layers "F.Cu" "B.Cu") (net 5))
 (via (at 139 113.4) (size 1.2) (drill 0.4) (layers "F.Cu" "B.Cu") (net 5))
 (via (at 147.6 123.6) (size 1.2) (drill 0.4) (layers "F.Cu" "B.Cu") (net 5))
 (via (at 146 117.8) (size 1.2) (drill 0.4) (layers "F.Cu" "B.Cu") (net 5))
 (segment (start 145.4 77.4) (end 128.23 77.4) (width 1.5) (layer "B.Cu") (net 5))
 (segment (start 150.8 109.8) (end 152.96 111.96) (width 1.5) (layer "B.Cu") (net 5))
 (segment (start 148.5 80.5) (end 150.8 82.8) (width 1.5) (layer "B.Cu") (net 5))
 (segment (start 150.8 82.8) (end 150.8 109.8) (width 1.5) (layer "B.Cu") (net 5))
 (segment (start 152.96 111.96) (end 153.945 111.96) (width 1.5) (layer "B.Cu") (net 5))
 (segment (start 146 122) (end 146 121.8) (width 1.5) (layer "B.Cu") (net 5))
 (segment (start 146 121.8) (end 146 117.8) (width 1.5) (layer "B.Cu") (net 5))
 (segment (start 147.6 123.6) (end 146 122) (width 1.5) (layer "B.Cu") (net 5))
 (segment (start 128.23 77.4) (end 127.145 78.485) (width 1.5) (layer "B.Cu") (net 5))
 (segment (start 148.5 80.5) (end 145.4 77.4) (width 1.5) (layer "B.Cu") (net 5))
 (segment (start 139 113.4) (end 139 105.38) (width 1.5) (layer "B.Cu") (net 5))
 (segment (start 106.735 127) (end 106.735 100.395) (width 1) (layer "F.Cu") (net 3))
 (segment (start 110.865 96.265) (end 101.745 96.265) (width 1) (layer "F.Cu") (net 3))
 (segment (start 106.735 100.395) (end 110.865 96.265) (width 1) (layer "F.Cu") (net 3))
 (segment (start 116.6 102) (end 110.865 96.265) (width 1) (layer "F.Cu") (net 3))
 (via (at 116.6 102) (size 0.8) (drill 0.4) (layers "F.Cu" "B.Cu") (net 3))
 (segment (start 116.6 106.85137) (end 116.6 102) (width 1) (layer "B.Cu") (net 3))
 (segment (start 130.36863 120.62) (end 116.6 106.85137) (width 1) (layer "B.Cu") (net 3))
 (segment (start 131.5 120.62) (end 130.36863 120.62) (width 1) (layer "B.Cu") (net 3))
 (segment (start 134.78 120.62) (end 130 125.4) (width 1) (layer "F.Cu") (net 17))
 (segment (start 139 120.62) (end 134.78 120.62) (width 1) (layer "F.Cu") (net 17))
 (via (at 130 125.4) (size 0.8) (drill 0.4) (layers "F.Cu" "B.Cu") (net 17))
 (segment (start 106.735 132.702081) (end 107.832919 133.8) (width 1) (layer "B.Cu") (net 17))
 (segment (start 114.2 115.2) (end 114.2 93.2) (width 1) (layer "B.Cu") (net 17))
 (segment (start 107.832919 133.8) (end 110.6 133.8) (width 1) (layer "B.Cu") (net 17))
 (segment (start 114.2 93.2) (end 109.645 88.645) (width 1) (layer "B.Cu") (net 17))
 (segment (start 112.6 116.8) (end 114.2 115.2) (width 1) (layer "B.Cu") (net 17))
 (segment (start 124.4 125.4) (end 114.2 115.2) (width 1) (layer "B.Cu") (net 17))
 (segment (start 109.645 88.645) (end 101.745 88.645) (width 1) (layer "B.Cu") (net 17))
 (segment (start 106.735 131.5) (end 106.735 132.702081) (width 1) (layer "B.Cu") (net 17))
 (segment (start 110.6 133.8) (end 112.6 131.8) (width 1) (layer "B.Cu") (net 17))
 (segment (start 130 125.4) (end 124.4 125.4) (width 1) (layer "B.Cu") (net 17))
 (segment (start 112.6 131.8) (end 112.6 116.8) (width 1) (layer "B.Cu") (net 17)))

